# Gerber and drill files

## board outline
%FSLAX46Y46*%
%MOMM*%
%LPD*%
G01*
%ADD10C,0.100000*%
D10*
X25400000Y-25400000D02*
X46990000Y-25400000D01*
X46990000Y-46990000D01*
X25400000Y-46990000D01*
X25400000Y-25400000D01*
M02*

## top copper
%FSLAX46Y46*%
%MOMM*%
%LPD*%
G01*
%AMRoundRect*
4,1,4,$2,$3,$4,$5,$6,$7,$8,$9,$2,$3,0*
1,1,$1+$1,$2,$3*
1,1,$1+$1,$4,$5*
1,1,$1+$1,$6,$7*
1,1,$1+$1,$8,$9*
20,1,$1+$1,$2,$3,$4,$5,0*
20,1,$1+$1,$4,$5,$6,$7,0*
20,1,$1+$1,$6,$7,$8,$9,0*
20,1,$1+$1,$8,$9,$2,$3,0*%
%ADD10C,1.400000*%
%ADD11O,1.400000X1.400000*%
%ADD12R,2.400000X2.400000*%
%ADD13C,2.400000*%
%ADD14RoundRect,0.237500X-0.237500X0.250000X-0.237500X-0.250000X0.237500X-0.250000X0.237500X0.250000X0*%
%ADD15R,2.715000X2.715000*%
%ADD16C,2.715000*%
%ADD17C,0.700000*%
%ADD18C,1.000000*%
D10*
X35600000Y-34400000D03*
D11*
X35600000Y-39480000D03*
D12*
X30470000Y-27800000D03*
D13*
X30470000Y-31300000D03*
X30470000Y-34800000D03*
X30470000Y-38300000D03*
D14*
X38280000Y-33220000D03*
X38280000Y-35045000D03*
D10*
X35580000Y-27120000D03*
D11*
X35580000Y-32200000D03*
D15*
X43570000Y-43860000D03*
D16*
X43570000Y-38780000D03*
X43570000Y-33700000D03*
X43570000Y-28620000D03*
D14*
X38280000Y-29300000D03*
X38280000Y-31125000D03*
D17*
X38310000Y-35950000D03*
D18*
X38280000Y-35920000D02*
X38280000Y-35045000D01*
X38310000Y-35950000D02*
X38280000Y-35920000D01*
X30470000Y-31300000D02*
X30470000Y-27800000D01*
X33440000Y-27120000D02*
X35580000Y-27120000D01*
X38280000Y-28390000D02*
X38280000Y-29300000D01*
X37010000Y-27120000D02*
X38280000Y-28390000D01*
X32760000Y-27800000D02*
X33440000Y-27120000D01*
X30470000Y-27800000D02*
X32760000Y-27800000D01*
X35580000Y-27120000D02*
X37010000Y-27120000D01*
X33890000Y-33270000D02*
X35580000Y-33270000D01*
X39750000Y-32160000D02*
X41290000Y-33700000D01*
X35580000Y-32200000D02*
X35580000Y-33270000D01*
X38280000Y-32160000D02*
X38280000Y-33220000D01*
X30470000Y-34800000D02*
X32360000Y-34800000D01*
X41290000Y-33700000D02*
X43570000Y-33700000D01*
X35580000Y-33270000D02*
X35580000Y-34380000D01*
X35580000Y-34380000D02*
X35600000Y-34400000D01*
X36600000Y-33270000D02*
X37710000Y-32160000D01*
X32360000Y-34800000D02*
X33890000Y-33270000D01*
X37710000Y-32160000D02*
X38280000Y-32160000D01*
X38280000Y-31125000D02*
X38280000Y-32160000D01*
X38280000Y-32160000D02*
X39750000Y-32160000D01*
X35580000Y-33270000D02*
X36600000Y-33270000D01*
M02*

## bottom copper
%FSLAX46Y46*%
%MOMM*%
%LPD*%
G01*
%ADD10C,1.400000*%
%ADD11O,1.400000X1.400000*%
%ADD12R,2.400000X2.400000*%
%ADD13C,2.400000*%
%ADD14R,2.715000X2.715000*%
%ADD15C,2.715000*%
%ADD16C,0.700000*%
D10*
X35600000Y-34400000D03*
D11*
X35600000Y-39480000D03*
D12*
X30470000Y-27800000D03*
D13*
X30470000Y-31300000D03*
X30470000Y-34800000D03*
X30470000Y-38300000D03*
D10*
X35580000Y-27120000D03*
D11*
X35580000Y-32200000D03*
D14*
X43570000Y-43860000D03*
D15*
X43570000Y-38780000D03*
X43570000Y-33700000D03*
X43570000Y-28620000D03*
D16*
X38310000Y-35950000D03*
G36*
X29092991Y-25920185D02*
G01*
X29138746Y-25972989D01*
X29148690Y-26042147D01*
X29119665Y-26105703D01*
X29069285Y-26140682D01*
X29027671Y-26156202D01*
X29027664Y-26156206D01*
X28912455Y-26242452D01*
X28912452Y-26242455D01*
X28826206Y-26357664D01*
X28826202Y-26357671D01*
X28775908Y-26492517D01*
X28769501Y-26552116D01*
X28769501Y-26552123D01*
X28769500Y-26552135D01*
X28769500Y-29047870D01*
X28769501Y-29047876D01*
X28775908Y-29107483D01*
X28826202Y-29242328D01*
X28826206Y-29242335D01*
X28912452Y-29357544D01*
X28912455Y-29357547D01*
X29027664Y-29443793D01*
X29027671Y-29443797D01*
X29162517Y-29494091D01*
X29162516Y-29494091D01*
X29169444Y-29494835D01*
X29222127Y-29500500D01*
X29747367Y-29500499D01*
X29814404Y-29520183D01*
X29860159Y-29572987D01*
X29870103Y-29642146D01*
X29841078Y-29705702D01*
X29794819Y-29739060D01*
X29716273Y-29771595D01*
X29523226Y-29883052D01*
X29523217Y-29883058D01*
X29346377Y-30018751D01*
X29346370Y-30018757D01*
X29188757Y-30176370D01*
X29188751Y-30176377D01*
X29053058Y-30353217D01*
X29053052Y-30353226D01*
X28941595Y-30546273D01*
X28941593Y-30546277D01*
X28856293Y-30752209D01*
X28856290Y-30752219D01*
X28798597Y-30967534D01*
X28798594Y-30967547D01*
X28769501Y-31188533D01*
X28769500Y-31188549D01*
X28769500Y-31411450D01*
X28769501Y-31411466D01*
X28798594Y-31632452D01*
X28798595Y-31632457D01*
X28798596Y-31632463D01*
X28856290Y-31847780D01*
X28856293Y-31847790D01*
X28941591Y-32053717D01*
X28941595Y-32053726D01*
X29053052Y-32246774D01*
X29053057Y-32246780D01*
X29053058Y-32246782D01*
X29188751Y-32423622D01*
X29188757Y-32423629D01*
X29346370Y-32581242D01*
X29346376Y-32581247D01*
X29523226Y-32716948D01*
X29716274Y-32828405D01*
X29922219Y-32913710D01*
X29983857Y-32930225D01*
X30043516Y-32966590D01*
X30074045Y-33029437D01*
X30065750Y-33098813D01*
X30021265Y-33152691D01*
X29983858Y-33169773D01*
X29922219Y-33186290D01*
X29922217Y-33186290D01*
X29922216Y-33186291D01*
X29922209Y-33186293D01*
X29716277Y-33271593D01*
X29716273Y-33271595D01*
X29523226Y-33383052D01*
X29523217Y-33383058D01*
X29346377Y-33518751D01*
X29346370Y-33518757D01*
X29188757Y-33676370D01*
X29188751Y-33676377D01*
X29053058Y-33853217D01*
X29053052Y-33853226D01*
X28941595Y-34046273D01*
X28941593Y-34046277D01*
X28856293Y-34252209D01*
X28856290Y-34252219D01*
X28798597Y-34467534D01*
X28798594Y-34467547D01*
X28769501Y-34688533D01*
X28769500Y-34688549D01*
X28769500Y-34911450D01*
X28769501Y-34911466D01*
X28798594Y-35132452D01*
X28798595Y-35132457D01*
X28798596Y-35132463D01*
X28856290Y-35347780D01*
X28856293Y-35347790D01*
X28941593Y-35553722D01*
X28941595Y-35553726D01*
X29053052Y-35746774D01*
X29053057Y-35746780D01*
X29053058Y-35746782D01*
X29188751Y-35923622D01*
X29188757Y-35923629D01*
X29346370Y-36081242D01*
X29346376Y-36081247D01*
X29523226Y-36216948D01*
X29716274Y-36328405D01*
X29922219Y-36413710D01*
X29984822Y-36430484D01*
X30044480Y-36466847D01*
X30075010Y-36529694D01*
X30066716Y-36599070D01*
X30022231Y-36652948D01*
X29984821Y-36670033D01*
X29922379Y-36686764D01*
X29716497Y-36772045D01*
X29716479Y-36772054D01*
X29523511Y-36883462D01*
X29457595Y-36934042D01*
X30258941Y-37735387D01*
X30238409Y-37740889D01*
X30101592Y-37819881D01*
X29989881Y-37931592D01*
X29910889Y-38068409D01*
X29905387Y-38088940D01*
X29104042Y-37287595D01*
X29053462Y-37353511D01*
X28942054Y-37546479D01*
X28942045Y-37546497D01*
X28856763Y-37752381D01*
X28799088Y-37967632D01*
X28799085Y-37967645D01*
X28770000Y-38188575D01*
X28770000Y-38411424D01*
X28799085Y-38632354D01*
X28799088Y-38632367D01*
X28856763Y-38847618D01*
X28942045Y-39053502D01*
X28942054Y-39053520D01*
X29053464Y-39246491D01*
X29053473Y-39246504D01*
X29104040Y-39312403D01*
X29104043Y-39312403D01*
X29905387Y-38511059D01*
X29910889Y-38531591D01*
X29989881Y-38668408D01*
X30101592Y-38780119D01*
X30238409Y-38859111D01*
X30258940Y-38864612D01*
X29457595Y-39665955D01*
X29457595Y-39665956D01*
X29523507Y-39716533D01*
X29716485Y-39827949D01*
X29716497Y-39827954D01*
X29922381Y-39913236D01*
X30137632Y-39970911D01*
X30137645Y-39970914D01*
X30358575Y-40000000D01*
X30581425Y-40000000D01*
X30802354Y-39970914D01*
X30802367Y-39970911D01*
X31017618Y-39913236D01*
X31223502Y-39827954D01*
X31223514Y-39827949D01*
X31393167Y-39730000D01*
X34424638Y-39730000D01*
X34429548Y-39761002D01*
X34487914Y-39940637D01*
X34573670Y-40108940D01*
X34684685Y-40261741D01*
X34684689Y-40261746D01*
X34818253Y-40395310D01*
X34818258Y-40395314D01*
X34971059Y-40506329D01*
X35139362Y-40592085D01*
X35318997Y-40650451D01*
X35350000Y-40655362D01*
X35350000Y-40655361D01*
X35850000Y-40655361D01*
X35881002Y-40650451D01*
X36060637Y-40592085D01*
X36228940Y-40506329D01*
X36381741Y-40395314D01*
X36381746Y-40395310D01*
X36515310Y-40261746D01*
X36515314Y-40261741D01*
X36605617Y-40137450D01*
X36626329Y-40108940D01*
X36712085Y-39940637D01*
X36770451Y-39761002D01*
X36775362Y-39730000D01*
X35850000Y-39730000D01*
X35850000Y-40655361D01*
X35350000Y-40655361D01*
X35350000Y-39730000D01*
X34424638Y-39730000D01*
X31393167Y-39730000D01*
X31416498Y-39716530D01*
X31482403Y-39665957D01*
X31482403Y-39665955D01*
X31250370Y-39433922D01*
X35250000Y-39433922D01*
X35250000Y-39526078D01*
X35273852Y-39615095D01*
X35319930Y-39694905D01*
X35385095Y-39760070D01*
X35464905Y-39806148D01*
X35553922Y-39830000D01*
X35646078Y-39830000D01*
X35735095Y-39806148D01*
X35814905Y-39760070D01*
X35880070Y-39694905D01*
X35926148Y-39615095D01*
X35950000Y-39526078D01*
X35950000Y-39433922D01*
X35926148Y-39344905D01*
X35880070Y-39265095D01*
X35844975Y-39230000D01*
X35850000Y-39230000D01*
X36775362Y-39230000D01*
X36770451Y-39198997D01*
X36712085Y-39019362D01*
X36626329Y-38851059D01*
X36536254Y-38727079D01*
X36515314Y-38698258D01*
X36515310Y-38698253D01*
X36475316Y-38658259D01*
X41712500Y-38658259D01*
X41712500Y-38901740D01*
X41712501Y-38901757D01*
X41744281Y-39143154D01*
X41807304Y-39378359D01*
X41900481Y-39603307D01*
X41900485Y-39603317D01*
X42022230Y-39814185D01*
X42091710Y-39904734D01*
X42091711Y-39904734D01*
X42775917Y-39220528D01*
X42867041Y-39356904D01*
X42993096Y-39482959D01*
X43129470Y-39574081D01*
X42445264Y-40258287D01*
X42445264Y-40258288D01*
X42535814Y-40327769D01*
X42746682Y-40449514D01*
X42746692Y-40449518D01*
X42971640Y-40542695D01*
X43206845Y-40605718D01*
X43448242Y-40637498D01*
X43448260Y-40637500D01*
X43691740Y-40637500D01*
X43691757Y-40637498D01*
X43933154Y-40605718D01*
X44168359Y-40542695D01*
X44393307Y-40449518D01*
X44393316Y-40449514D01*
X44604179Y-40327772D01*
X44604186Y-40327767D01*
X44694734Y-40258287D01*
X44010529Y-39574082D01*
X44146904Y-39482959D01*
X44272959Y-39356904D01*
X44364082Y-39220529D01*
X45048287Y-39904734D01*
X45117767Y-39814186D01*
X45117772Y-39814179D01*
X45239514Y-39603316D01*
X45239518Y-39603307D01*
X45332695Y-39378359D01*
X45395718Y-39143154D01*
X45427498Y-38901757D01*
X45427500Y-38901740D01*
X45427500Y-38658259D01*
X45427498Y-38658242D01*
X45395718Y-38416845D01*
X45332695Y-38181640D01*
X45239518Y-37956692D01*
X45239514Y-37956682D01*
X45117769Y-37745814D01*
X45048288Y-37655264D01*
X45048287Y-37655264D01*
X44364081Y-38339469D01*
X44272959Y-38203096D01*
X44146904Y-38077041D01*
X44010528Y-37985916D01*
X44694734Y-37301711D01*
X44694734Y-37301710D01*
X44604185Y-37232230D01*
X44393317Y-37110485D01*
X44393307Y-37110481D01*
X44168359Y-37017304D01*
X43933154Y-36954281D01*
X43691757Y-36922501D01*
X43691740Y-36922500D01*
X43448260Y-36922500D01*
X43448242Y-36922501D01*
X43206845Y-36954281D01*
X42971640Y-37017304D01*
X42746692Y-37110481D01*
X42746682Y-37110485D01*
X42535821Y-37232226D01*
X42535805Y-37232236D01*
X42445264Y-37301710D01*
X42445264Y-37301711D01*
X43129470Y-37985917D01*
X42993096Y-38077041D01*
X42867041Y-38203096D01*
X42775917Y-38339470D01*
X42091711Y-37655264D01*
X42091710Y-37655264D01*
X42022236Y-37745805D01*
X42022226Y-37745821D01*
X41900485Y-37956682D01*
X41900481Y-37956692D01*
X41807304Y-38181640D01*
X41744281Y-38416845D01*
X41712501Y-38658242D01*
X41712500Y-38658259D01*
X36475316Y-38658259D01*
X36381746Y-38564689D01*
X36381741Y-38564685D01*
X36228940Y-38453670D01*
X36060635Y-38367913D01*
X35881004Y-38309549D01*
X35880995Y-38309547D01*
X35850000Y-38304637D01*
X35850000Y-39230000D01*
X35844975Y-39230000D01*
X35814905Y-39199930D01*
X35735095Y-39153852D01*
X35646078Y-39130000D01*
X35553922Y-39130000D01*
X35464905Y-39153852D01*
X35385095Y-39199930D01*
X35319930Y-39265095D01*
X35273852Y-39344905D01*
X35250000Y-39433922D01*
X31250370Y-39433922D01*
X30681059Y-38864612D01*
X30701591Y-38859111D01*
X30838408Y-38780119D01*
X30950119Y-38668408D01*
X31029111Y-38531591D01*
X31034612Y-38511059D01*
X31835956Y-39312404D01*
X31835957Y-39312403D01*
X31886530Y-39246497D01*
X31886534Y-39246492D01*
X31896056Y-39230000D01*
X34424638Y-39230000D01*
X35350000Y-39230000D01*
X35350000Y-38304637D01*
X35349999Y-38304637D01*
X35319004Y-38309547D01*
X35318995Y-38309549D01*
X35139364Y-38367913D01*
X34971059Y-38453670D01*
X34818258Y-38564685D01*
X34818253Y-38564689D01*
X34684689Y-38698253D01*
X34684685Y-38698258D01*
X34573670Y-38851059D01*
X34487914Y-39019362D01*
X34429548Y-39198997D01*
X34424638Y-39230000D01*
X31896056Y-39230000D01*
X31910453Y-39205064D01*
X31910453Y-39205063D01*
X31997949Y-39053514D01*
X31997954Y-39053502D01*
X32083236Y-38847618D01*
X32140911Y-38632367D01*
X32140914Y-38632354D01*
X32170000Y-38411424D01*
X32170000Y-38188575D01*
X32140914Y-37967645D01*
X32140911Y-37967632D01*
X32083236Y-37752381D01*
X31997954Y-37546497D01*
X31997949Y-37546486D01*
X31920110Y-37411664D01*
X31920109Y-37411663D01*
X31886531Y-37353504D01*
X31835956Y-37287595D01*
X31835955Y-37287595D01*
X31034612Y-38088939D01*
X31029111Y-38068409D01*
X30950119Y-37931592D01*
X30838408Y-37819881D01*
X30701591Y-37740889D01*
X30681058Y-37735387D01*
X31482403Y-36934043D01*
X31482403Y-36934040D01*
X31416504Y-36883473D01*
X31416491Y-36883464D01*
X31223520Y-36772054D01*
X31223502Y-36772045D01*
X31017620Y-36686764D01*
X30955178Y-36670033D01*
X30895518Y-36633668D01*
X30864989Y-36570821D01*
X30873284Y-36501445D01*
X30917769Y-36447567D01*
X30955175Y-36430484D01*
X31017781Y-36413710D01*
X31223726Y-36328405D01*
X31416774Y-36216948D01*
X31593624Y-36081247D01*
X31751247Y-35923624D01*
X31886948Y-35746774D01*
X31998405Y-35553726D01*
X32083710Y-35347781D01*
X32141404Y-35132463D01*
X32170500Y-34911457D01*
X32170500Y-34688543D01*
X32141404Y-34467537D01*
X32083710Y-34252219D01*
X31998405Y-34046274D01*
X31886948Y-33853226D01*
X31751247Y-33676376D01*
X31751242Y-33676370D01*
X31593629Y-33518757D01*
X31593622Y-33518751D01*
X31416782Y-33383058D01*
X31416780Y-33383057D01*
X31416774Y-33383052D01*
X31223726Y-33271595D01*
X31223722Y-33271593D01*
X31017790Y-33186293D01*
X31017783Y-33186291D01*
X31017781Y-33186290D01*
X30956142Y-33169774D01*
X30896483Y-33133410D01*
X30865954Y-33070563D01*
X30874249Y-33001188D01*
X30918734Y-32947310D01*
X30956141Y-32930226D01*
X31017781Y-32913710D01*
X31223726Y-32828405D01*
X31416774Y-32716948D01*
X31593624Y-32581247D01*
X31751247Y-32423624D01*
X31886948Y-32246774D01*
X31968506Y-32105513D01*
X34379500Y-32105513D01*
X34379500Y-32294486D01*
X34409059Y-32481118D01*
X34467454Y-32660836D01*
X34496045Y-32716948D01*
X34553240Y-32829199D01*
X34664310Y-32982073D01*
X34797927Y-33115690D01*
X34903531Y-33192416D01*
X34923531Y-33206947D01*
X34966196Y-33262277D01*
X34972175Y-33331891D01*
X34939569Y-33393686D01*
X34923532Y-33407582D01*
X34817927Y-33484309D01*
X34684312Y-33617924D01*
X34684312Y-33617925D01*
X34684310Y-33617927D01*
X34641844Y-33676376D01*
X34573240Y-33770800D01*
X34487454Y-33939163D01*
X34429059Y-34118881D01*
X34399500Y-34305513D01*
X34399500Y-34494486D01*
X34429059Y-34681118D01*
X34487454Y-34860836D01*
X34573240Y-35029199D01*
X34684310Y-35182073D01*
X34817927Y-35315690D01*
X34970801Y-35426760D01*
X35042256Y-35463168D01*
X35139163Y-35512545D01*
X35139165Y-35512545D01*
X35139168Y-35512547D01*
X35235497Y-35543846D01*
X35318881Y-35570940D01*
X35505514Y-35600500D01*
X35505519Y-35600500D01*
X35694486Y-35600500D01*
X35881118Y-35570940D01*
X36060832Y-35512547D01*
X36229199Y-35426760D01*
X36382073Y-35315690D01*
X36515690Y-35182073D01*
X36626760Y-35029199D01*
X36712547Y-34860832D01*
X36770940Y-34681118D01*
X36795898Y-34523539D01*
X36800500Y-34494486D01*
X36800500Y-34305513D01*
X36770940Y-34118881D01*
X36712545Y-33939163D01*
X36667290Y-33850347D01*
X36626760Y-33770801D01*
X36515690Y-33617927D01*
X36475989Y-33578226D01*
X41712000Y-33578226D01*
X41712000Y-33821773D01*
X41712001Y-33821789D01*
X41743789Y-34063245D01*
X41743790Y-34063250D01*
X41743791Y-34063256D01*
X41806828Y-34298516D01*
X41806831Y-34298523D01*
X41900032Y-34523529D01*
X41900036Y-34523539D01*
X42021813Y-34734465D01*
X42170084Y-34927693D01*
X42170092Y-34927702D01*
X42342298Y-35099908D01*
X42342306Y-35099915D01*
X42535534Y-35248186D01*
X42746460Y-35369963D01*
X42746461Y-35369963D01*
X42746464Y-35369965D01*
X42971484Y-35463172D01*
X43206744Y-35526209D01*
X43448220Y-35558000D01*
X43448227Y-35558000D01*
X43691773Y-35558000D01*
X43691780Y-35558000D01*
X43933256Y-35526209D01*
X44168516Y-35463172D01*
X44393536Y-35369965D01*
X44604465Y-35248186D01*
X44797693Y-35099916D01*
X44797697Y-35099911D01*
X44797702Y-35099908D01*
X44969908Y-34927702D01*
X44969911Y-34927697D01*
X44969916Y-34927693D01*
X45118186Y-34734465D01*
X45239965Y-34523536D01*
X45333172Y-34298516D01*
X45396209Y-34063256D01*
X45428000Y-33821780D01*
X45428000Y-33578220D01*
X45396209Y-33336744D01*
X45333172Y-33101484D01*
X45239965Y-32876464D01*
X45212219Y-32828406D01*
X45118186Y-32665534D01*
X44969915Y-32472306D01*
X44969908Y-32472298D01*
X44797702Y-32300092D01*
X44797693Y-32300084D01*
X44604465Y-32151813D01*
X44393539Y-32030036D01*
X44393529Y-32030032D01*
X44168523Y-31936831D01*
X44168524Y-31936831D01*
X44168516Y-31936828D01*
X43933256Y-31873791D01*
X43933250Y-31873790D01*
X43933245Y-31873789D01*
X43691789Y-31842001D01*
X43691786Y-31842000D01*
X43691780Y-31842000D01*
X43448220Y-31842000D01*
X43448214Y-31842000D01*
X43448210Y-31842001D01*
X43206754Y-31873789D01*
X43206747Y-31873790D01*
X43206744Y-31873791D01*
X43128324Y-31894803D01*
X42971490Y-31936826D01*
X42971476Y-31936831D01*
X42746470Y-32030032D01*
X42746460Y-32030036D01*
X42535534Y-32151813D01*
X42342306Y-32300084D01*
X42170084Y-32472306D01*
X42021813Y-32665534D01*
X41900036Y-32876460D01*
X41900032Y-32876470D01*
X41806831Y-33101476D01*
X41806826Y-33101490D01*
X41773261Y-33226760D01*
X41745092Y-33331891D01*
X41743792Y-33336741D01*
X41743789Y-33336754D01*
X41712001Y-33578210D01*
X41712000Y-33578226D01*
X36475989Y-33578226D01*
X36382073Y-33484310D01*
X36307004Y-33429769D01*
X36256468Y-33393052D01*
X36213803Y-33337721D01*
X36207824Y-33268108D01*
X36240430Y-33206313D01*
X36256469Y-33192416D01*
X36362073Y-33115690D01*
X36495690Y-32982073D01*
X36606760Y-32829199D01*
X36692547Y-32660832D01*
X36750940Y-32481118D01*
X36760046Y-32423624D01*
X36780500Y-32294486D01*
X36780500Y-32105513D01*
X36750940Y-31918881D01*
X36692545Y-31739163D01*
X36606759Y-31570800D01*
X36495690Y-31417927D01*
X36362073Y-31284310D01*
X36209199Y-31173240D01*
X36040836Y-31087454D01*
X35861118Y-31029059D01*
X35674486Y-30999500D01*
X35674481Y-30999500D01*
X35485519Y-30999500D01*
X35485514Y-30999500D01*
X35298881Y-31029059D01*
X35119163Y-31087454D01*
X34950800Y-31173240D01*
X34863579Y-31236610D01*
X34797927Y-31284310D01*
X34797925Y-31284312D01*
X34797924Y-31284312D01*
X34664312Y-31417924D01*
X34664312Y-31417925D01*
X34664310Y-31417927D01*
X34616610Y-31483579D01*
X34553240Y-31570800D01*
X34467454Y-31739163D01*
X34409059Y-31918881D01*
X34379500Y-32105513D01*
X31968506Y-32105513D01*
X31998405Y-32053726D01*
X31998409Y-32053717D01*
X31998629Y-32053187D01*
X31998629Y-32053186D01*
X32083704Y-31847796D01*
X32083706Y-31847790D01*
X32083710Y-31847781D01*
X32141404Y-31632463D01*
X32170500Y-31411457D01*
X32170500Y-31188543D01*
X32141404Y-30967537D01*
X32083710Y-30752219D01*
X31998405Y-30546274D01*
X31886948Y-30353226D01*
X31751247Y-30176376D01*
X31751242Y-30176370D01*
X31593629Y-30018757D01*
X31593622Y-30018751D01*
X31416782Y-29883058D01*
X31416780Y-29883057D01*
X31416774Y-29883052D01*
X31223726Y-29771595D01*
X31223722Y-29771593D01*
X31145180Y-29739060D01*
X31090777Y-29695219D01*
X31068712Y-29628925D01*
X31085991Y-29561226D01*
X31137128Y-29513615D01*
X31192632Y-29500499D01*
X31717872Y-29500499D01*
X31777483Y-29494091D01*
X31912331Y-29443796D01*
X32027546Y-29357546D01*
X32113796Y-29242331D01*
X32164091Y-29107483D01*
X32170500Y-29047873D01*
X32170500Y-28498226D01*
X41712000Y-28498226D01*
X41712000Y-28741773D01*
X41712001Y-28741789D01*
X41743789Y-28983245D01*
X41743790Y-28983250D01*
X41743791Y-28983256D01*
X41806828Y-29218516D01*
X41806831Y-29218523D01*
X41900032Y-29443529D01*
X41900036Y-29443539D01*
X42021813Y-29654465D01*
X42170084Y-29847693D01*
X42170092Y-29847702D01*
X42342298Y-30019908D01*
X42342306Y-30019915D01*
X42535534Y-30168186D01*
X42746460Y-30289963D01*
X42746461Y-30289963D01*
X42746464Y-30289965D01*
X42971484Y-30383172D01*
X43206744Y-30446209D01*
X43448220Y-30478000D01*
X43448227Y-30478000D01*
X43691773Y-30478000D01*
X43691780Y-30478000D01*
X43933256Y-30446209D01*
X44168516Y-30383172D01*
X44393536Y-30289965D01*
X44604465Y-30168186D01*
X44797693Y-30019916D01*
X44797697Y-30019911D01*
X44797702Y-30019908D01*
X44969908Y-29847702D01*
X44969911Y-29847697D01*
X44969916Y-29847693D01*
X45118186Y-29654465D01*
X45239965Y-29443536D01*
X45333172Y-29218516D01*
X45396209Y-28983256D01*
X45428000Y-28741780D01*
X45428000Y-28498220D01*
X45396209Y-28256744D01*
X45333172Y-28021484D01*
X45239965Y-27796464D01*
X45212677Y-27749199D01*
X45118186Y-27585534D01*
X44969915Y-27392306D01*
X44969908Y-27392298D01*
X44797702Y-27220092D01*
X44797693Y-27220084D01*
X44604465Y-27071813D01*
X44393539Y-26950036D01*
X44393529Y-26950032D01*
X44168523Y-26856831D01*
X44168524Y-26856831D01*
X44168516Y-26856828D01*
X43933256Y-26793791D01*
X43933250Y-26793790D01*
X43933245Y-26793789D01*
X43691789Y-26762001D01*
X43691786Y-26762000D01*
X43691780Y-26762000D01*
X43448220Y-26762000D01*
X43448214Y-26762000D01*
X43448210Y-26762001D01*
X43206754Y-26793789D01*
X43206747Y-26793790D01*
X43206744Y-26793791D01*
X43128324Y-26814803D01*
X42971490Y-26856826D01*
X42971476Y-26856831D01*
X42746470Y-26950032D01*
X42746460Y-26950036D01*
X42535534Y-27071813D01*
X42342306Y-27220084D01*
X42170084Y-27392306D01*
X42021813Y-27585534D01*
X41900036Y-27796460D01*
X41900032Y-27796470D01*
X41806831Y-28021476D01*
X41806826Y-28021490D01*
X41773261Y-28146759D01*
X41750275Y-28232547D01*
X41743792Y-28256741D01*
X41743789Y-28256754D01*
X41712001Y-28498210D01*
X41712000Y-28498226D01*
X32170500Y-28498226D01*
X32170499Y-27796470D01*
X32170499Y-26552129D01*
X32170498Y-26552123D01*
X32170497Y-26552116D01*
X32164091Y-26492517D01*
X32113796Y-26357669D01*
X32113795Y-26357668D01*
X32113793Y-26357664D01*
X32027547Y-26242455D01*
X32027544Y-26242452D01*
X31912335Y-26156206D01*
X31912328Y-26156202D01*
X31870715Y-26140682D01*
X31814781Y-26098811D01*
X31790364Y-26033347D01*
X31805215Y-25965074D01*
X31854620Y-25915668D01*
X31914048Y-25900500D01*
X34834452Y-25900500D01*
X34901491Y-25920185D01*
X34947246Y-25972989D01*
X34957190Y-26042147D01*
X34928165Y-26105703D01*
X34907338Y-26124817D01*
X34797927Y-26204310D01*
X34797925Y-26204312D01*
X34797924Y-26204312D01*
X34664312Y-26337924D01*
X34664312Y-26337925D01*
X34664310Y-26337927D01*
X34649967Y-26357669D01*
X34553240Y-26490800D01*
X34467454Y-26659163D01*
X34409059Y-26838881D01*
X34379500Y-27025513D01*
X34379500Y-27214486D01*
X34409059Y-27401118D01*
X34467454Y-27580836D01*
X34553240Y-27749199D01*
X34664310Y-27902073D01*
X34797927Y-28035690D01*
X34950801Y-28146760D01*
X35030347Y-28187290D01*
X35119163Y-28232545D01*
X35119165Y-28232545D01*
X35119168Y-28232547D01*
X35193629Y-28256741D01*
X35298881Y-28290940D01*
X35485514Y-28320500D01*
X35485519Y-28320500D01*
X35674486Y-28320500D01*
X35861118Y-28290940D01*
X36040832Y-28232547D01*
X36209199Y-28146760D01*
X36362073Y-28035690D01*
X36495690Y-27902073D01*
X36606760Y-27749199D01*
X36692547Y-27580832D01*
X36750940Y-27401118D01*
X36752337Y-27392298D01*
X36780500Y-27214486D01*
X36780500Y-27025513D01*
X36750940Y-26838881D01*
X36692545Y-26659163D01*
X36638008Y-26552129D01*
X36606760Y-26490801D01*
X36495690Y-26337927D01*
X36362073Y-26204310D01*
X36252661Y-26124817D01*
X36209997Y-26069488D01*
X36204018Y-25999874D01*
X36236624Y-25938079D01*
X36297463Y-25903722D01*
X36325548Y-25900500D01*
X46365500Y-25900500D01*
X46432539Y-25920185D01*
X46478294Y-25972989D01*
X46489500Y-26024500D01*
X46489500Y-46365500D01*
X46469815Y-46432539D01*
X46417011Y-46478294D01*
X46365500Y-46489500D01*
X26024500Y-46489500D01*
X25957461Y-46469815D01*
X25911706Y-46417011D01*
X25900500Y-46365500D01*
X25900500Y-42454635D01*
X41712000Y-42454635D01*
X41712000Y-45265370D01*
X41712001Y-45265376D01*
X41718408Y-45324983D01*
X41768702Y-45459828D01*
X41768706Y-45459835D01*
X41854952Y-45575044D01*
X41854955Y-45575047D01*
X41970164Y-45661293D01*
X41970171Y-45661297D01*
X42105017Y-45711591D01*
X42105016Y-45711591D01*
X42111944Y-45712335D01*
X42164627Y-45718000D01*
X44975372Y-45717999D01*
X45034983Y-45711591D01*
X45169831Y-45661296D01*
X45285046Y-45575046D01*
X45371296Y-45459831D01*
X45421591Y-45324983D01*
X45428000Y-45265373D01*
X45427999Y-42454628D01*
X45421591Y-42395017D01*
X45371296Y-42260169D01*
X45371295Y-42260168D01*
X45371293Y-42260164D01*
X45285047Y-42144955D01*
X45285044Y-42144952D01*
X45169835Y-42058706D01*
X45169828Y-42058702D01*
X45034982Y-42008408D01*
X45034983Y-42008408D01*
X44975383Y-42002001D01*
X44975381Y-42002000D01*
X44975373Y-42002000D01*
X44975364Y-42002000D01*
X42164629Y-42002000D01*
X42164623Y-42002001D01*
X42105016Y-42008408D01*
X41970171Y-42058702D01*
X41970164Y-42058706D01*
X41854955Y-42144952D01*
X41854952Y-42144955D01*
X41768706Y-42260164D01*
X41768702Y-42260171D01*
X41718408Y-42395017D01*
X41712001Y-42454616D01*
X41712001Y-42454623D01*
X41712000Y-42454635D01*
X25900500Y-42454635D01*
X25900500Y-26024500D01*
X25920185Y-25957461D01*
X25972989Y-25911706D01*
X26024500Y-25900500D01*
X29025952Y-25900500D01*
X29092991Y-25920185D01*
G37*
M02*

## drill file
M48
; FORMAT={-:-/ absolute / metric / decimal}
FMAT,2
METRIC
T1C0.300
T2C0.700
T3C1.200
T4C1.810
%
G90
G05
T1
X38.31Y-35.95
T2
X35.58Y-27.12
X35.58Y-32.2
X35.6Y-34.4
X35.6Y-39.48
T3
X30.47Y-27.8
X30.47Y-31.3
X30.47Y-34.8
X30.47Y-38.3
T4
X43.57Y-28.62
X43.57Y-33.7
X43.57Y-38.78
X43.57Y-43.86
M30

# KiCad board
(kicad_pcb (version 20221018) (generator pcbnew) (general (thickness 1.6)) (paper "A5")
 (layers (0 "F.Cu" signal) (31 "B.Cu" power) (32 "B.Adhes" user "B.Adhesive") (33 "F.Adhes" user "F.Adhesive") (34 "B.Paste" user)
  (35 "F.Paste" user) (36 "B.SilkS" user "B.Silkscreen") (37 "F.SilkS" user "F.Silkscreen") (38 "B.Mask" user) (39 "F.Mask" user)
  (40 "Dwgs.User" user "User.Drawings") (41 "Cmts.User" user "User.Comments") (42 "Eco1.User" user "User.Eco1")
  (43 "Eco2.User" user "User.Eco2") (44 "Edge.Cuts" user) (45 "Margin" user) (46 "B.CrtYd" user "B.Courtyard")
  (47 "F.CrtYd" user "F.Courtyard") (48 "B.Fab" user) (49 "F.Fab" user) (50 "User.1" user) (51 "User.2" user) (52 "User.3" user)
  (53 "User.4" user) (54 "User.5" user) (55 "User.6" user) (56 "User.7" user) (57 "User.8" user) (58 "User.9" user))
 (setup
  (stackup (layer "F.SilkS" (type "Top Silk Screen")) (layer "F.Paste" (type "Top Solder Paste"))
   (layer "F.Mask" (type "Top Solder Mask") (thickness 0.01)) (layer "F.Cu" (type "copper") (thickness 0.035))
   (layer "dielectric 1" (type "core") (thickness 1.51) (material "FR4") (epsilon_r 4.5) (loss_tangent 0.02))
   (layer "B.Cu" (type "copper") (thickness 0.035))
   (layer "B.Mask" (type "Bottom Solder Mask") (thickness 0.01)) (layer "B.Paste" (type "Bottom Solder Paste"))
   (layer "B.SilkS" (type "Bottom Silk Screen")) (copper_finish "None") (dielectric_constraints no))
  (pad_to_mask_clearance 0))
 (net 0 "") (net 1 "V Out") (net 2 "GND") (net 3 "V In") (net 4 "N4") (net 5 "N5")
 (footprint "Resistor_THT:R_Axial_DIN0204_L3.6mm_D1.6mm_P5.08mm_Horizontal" (layer "F.Cu") (at 35.6 34.4 -90)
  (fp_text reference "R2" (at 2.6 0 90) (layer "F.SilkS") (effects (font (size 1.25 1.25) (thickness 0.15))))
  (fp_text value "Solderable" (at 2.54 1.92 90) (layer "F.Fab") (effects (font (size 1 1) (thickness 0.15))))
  (pad "1" thru_hole circle (at 0 0 270) (size 1.4 1.4) (drill 0.7) (layers "*.Cu" "*.Mask") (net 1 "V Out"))
  (pad "2" thru_hole oval (at 5.08 0 270) (size 1.4 1.4) (drill 0.7) (layers "*.Cu" "*.Mask") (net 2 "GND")))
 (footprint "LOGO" (layer "F.Cu") (at 34.197606 42.341825 -90)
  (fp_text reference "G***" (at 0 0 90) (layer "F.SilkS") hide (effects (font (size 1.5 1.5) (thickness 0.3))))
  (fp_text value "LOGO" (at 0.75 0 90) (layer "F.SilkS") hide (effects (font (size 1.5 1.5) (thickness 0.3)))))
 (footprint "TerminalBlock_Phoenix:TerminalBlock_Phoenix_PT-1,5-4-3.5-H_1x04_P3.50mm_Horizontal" (layer "F.Cu") (at 30.47 27.8 -90)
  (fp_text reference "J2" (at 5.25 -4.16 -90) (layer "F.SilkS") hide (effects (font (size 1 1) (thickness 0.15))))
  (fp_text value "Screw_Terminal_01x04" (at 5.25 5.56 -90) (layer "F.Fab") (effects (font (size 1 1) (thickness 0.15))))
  (pad "1" thru_hole rect (at 0 0 270) (size 2.4 2.4) (drill 1.2) (layers "*.Cu" "*.Mask") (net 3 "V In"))
  (pad "2" thru_hole circle (at 3.5 0 270) (size 2.4 2.4) (drill 1.2) (layers "*.Cu" "*.Mask") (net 3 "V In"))
  (pad "3" thru_hole circle (at 7 0 270) (size 2.4 2.4) (drill 1.2) (layers "*.Cu" "*.Mask") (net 1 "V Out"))
  (pad "4" thru_hole circle (at 10.5 0 270) (size 2.4 2.4) (drill 1.2) (layers "*.Cu" "*.Mask") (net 2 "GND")))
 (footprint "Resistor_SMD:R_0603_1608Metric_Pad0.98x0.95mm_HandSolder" (layer "F.Cu") (at 38.28 34.1325 -90)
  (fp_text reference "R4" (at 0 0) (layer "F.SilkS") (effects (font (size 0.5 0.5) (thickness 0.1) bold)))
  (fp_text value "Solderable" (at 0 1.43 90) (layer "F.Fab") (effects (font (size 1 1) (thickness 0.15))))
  (pad "1" smd roundrect (at -0.9125 0 270) (size 0.975 0.95) (layers "F.Cu" "F.Paste" "F.Mask") (roundrect_rratio 0.25) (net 1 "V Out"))
  (pad "2" smd roundrect (at 0.9125 0 270) (size 0.975 0.95) (layers "F.Cu" "F.Paste" "F.Mask") (roundrect_rratio 0.25) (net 2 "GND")))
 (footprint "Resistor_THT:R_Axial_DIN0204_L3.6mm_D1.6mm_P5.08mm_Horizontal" (layer "F.Cu") (at 35.58 27.12 -90)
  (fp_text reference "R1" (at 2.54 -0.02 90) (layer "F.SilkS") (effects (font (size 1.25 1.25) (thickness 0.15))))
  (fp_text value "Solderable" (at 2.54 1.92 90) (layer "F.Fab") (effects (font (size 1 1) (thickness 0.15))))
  (pad "1" thru_hole circle (at 0 0 270) (size 1.4 1.4) (drill 0.7) (layers "*.Cu" "*.Mask") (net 3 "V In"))
  (pad "2" thru_hole oval (at 5.08 0 270) (size 1.4 1.4) (drill 0.7) (layers "*.Cu" "*.Mask") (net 1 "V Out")))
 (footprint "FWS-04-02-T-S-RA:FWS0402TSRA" (layer "F.Cu") (at 43.57 43.86 -90)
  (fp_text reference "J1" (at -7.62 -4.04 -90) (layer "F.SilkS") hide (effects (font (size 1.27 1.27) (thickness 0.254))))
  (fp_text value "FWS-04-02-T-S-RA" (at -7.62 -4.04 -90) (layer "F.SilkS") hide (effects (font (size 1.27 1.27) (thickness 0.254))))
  (pad "1" thru_hole rect (at 0 0 270) (size 2.715 2.715) (drill 1.81) (layers "*.Cu" "*.Mask") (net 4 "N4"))
  (pad "2" thru_hole circle (at -5.08 0 270) (size 2.715 2.715) (drill 1.81) (layers "*.Cu" "*.Mask") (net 2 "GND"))
  (pad "3" thru_hole circle (at -10.16 0 270) (size 2.715 2.715) (drill 1.81) (layers "*.Cu" "*.Mask") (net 1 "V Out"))
  (pad "4" thru_hole circle (at -15.24 0 270) (size 2.715 2.715) (drill 1.81) (layers "*.Cu" "*.Mask") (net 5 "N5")))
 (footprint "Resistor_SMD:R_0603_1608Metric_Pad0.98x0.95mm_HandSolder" (layer "F.Cu") (at 38.28 30.2125 -90)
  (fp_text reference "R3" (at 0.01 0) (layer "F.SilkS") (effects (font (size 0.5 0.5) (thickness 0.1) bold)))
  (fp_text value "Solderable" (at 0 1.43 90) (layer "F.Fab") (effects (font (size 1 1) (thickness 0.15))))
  (pad "1" smd roundrect (at -0.9125 0 270) (size 0.975 0.95) (layers "F.Cu" "F.Paste" "F.Mask") (roundrect_rratio 0.25) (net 3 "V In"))
  (pad "2" smd roundrect (at 0.9125 0 270) (size 0.975 0.95) (layers "F.Cu" "F.Paste" "F.Mask") (roundrect_rratio 0.25) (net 1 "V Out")))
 (gr_rect (start 25.4 25.4) (end 46.99 46.99) (stroke (width 0.1) (type default)) (fill none) (layer "Edge.Cuts"))
 (segment (start 38.28 35.92) (end 38.28 35.045) (width 1) (layer "F.Cu") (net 2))
 (segment (start 38.31 35.95) (end 38.28 35.92) (width 1) (layer "F.Cu") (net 2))
 (via (at 38.31 35.95) (size 0.7) (drill 0.3) (layers "F.Cu" "B.Cu") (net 2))
 (segment (start 30.47 31.3) (end 30.47 27.8) (width 1) (layer "F.Cu") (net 3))
 (segment (start 33.44 27.12) (end 35.58 27.12) (width 1) (layer "F.Cu") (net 3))
 (segment (start 38.28 28.39) (end 38.28 29.3) (width 1) (layer "F.Cu") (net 3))
 (segment (start 37.01 27.12) (end 38.28 28.39) (width 1) (layer "F.Cu") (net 3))
 (segment (start 32.76 27.8) (end 33.44 27.12) (width 1) (layer "F.Cu") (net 3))
 (segment (start 30.47 27.8) (end 32.76 27.8) (width 1) (layer "F.Cu") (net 3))
 (segment (start 35.58 27.12) (end 37.01 27.12) (width 1) (layer "F.Cu") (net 3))
 (segment (start 33.89 33.27) (end 35.58 33.27) (width 1) (layer "F.Cu") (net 1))
 (segment (start 39.75 32.16) (end 41.29 33.7) (width 1) (layer "F.Cu") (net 1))
 (segment (start 35.58 32.2) (end 35.58 33.27) (width 1) (layer "F.Cu") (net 1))
 (segment (start 38.28 32.16) (end 38.28 33.22) (width 1) (layer "F.Cu") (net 1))
 (segment (start 30.47 34.8) (end 32.36 34.8) (width 1) (layer "F.Cu") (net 1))
 (segment (start 41.29 33.7) (end 43.57 33.7) (width 1) (layer "F.Cu") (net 1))
 (segment (start 35.58 33.27) (end 35.58 34.38) (width 1) (layer "F.Cu") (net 1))
 (segment (start 35.58 34.38) (end 35.6 34.4) (width 1) (layer "F.Cu") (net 1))
 (segment (start 36.6 33.27) (end 37.71 32.16) (width 1) (layer "F.Cu") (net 1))
 (segment (start 32.36 34.8) (end 33.89 33.27) (width 1) (layer "F.Cu") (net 1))
 (segment (start 37.71 32.16) (end 38.28 32.16) (width 1) (layer "F.Cu") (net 1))
 (segment (start 38.28 31.125) (end 38.28 32.16) (width 1) (layer "F.Cu") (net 1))
 (segment (start 38.28 32.16) (end 39.75 32.16) (width 1) (layer "F.Cu") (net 1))
 (segment (start 35.58 33.27) (end 36.6 33.27) (width 1) (layer "F.Cu") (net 1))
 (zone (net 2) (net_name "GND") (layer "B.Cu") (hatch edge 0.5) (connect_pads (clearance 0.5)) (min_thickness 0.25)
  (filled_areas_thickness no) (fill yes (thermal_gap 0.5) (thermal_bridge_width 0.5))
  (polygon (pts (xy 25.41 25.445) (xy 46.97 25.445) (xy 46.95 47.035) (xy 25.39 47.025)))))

